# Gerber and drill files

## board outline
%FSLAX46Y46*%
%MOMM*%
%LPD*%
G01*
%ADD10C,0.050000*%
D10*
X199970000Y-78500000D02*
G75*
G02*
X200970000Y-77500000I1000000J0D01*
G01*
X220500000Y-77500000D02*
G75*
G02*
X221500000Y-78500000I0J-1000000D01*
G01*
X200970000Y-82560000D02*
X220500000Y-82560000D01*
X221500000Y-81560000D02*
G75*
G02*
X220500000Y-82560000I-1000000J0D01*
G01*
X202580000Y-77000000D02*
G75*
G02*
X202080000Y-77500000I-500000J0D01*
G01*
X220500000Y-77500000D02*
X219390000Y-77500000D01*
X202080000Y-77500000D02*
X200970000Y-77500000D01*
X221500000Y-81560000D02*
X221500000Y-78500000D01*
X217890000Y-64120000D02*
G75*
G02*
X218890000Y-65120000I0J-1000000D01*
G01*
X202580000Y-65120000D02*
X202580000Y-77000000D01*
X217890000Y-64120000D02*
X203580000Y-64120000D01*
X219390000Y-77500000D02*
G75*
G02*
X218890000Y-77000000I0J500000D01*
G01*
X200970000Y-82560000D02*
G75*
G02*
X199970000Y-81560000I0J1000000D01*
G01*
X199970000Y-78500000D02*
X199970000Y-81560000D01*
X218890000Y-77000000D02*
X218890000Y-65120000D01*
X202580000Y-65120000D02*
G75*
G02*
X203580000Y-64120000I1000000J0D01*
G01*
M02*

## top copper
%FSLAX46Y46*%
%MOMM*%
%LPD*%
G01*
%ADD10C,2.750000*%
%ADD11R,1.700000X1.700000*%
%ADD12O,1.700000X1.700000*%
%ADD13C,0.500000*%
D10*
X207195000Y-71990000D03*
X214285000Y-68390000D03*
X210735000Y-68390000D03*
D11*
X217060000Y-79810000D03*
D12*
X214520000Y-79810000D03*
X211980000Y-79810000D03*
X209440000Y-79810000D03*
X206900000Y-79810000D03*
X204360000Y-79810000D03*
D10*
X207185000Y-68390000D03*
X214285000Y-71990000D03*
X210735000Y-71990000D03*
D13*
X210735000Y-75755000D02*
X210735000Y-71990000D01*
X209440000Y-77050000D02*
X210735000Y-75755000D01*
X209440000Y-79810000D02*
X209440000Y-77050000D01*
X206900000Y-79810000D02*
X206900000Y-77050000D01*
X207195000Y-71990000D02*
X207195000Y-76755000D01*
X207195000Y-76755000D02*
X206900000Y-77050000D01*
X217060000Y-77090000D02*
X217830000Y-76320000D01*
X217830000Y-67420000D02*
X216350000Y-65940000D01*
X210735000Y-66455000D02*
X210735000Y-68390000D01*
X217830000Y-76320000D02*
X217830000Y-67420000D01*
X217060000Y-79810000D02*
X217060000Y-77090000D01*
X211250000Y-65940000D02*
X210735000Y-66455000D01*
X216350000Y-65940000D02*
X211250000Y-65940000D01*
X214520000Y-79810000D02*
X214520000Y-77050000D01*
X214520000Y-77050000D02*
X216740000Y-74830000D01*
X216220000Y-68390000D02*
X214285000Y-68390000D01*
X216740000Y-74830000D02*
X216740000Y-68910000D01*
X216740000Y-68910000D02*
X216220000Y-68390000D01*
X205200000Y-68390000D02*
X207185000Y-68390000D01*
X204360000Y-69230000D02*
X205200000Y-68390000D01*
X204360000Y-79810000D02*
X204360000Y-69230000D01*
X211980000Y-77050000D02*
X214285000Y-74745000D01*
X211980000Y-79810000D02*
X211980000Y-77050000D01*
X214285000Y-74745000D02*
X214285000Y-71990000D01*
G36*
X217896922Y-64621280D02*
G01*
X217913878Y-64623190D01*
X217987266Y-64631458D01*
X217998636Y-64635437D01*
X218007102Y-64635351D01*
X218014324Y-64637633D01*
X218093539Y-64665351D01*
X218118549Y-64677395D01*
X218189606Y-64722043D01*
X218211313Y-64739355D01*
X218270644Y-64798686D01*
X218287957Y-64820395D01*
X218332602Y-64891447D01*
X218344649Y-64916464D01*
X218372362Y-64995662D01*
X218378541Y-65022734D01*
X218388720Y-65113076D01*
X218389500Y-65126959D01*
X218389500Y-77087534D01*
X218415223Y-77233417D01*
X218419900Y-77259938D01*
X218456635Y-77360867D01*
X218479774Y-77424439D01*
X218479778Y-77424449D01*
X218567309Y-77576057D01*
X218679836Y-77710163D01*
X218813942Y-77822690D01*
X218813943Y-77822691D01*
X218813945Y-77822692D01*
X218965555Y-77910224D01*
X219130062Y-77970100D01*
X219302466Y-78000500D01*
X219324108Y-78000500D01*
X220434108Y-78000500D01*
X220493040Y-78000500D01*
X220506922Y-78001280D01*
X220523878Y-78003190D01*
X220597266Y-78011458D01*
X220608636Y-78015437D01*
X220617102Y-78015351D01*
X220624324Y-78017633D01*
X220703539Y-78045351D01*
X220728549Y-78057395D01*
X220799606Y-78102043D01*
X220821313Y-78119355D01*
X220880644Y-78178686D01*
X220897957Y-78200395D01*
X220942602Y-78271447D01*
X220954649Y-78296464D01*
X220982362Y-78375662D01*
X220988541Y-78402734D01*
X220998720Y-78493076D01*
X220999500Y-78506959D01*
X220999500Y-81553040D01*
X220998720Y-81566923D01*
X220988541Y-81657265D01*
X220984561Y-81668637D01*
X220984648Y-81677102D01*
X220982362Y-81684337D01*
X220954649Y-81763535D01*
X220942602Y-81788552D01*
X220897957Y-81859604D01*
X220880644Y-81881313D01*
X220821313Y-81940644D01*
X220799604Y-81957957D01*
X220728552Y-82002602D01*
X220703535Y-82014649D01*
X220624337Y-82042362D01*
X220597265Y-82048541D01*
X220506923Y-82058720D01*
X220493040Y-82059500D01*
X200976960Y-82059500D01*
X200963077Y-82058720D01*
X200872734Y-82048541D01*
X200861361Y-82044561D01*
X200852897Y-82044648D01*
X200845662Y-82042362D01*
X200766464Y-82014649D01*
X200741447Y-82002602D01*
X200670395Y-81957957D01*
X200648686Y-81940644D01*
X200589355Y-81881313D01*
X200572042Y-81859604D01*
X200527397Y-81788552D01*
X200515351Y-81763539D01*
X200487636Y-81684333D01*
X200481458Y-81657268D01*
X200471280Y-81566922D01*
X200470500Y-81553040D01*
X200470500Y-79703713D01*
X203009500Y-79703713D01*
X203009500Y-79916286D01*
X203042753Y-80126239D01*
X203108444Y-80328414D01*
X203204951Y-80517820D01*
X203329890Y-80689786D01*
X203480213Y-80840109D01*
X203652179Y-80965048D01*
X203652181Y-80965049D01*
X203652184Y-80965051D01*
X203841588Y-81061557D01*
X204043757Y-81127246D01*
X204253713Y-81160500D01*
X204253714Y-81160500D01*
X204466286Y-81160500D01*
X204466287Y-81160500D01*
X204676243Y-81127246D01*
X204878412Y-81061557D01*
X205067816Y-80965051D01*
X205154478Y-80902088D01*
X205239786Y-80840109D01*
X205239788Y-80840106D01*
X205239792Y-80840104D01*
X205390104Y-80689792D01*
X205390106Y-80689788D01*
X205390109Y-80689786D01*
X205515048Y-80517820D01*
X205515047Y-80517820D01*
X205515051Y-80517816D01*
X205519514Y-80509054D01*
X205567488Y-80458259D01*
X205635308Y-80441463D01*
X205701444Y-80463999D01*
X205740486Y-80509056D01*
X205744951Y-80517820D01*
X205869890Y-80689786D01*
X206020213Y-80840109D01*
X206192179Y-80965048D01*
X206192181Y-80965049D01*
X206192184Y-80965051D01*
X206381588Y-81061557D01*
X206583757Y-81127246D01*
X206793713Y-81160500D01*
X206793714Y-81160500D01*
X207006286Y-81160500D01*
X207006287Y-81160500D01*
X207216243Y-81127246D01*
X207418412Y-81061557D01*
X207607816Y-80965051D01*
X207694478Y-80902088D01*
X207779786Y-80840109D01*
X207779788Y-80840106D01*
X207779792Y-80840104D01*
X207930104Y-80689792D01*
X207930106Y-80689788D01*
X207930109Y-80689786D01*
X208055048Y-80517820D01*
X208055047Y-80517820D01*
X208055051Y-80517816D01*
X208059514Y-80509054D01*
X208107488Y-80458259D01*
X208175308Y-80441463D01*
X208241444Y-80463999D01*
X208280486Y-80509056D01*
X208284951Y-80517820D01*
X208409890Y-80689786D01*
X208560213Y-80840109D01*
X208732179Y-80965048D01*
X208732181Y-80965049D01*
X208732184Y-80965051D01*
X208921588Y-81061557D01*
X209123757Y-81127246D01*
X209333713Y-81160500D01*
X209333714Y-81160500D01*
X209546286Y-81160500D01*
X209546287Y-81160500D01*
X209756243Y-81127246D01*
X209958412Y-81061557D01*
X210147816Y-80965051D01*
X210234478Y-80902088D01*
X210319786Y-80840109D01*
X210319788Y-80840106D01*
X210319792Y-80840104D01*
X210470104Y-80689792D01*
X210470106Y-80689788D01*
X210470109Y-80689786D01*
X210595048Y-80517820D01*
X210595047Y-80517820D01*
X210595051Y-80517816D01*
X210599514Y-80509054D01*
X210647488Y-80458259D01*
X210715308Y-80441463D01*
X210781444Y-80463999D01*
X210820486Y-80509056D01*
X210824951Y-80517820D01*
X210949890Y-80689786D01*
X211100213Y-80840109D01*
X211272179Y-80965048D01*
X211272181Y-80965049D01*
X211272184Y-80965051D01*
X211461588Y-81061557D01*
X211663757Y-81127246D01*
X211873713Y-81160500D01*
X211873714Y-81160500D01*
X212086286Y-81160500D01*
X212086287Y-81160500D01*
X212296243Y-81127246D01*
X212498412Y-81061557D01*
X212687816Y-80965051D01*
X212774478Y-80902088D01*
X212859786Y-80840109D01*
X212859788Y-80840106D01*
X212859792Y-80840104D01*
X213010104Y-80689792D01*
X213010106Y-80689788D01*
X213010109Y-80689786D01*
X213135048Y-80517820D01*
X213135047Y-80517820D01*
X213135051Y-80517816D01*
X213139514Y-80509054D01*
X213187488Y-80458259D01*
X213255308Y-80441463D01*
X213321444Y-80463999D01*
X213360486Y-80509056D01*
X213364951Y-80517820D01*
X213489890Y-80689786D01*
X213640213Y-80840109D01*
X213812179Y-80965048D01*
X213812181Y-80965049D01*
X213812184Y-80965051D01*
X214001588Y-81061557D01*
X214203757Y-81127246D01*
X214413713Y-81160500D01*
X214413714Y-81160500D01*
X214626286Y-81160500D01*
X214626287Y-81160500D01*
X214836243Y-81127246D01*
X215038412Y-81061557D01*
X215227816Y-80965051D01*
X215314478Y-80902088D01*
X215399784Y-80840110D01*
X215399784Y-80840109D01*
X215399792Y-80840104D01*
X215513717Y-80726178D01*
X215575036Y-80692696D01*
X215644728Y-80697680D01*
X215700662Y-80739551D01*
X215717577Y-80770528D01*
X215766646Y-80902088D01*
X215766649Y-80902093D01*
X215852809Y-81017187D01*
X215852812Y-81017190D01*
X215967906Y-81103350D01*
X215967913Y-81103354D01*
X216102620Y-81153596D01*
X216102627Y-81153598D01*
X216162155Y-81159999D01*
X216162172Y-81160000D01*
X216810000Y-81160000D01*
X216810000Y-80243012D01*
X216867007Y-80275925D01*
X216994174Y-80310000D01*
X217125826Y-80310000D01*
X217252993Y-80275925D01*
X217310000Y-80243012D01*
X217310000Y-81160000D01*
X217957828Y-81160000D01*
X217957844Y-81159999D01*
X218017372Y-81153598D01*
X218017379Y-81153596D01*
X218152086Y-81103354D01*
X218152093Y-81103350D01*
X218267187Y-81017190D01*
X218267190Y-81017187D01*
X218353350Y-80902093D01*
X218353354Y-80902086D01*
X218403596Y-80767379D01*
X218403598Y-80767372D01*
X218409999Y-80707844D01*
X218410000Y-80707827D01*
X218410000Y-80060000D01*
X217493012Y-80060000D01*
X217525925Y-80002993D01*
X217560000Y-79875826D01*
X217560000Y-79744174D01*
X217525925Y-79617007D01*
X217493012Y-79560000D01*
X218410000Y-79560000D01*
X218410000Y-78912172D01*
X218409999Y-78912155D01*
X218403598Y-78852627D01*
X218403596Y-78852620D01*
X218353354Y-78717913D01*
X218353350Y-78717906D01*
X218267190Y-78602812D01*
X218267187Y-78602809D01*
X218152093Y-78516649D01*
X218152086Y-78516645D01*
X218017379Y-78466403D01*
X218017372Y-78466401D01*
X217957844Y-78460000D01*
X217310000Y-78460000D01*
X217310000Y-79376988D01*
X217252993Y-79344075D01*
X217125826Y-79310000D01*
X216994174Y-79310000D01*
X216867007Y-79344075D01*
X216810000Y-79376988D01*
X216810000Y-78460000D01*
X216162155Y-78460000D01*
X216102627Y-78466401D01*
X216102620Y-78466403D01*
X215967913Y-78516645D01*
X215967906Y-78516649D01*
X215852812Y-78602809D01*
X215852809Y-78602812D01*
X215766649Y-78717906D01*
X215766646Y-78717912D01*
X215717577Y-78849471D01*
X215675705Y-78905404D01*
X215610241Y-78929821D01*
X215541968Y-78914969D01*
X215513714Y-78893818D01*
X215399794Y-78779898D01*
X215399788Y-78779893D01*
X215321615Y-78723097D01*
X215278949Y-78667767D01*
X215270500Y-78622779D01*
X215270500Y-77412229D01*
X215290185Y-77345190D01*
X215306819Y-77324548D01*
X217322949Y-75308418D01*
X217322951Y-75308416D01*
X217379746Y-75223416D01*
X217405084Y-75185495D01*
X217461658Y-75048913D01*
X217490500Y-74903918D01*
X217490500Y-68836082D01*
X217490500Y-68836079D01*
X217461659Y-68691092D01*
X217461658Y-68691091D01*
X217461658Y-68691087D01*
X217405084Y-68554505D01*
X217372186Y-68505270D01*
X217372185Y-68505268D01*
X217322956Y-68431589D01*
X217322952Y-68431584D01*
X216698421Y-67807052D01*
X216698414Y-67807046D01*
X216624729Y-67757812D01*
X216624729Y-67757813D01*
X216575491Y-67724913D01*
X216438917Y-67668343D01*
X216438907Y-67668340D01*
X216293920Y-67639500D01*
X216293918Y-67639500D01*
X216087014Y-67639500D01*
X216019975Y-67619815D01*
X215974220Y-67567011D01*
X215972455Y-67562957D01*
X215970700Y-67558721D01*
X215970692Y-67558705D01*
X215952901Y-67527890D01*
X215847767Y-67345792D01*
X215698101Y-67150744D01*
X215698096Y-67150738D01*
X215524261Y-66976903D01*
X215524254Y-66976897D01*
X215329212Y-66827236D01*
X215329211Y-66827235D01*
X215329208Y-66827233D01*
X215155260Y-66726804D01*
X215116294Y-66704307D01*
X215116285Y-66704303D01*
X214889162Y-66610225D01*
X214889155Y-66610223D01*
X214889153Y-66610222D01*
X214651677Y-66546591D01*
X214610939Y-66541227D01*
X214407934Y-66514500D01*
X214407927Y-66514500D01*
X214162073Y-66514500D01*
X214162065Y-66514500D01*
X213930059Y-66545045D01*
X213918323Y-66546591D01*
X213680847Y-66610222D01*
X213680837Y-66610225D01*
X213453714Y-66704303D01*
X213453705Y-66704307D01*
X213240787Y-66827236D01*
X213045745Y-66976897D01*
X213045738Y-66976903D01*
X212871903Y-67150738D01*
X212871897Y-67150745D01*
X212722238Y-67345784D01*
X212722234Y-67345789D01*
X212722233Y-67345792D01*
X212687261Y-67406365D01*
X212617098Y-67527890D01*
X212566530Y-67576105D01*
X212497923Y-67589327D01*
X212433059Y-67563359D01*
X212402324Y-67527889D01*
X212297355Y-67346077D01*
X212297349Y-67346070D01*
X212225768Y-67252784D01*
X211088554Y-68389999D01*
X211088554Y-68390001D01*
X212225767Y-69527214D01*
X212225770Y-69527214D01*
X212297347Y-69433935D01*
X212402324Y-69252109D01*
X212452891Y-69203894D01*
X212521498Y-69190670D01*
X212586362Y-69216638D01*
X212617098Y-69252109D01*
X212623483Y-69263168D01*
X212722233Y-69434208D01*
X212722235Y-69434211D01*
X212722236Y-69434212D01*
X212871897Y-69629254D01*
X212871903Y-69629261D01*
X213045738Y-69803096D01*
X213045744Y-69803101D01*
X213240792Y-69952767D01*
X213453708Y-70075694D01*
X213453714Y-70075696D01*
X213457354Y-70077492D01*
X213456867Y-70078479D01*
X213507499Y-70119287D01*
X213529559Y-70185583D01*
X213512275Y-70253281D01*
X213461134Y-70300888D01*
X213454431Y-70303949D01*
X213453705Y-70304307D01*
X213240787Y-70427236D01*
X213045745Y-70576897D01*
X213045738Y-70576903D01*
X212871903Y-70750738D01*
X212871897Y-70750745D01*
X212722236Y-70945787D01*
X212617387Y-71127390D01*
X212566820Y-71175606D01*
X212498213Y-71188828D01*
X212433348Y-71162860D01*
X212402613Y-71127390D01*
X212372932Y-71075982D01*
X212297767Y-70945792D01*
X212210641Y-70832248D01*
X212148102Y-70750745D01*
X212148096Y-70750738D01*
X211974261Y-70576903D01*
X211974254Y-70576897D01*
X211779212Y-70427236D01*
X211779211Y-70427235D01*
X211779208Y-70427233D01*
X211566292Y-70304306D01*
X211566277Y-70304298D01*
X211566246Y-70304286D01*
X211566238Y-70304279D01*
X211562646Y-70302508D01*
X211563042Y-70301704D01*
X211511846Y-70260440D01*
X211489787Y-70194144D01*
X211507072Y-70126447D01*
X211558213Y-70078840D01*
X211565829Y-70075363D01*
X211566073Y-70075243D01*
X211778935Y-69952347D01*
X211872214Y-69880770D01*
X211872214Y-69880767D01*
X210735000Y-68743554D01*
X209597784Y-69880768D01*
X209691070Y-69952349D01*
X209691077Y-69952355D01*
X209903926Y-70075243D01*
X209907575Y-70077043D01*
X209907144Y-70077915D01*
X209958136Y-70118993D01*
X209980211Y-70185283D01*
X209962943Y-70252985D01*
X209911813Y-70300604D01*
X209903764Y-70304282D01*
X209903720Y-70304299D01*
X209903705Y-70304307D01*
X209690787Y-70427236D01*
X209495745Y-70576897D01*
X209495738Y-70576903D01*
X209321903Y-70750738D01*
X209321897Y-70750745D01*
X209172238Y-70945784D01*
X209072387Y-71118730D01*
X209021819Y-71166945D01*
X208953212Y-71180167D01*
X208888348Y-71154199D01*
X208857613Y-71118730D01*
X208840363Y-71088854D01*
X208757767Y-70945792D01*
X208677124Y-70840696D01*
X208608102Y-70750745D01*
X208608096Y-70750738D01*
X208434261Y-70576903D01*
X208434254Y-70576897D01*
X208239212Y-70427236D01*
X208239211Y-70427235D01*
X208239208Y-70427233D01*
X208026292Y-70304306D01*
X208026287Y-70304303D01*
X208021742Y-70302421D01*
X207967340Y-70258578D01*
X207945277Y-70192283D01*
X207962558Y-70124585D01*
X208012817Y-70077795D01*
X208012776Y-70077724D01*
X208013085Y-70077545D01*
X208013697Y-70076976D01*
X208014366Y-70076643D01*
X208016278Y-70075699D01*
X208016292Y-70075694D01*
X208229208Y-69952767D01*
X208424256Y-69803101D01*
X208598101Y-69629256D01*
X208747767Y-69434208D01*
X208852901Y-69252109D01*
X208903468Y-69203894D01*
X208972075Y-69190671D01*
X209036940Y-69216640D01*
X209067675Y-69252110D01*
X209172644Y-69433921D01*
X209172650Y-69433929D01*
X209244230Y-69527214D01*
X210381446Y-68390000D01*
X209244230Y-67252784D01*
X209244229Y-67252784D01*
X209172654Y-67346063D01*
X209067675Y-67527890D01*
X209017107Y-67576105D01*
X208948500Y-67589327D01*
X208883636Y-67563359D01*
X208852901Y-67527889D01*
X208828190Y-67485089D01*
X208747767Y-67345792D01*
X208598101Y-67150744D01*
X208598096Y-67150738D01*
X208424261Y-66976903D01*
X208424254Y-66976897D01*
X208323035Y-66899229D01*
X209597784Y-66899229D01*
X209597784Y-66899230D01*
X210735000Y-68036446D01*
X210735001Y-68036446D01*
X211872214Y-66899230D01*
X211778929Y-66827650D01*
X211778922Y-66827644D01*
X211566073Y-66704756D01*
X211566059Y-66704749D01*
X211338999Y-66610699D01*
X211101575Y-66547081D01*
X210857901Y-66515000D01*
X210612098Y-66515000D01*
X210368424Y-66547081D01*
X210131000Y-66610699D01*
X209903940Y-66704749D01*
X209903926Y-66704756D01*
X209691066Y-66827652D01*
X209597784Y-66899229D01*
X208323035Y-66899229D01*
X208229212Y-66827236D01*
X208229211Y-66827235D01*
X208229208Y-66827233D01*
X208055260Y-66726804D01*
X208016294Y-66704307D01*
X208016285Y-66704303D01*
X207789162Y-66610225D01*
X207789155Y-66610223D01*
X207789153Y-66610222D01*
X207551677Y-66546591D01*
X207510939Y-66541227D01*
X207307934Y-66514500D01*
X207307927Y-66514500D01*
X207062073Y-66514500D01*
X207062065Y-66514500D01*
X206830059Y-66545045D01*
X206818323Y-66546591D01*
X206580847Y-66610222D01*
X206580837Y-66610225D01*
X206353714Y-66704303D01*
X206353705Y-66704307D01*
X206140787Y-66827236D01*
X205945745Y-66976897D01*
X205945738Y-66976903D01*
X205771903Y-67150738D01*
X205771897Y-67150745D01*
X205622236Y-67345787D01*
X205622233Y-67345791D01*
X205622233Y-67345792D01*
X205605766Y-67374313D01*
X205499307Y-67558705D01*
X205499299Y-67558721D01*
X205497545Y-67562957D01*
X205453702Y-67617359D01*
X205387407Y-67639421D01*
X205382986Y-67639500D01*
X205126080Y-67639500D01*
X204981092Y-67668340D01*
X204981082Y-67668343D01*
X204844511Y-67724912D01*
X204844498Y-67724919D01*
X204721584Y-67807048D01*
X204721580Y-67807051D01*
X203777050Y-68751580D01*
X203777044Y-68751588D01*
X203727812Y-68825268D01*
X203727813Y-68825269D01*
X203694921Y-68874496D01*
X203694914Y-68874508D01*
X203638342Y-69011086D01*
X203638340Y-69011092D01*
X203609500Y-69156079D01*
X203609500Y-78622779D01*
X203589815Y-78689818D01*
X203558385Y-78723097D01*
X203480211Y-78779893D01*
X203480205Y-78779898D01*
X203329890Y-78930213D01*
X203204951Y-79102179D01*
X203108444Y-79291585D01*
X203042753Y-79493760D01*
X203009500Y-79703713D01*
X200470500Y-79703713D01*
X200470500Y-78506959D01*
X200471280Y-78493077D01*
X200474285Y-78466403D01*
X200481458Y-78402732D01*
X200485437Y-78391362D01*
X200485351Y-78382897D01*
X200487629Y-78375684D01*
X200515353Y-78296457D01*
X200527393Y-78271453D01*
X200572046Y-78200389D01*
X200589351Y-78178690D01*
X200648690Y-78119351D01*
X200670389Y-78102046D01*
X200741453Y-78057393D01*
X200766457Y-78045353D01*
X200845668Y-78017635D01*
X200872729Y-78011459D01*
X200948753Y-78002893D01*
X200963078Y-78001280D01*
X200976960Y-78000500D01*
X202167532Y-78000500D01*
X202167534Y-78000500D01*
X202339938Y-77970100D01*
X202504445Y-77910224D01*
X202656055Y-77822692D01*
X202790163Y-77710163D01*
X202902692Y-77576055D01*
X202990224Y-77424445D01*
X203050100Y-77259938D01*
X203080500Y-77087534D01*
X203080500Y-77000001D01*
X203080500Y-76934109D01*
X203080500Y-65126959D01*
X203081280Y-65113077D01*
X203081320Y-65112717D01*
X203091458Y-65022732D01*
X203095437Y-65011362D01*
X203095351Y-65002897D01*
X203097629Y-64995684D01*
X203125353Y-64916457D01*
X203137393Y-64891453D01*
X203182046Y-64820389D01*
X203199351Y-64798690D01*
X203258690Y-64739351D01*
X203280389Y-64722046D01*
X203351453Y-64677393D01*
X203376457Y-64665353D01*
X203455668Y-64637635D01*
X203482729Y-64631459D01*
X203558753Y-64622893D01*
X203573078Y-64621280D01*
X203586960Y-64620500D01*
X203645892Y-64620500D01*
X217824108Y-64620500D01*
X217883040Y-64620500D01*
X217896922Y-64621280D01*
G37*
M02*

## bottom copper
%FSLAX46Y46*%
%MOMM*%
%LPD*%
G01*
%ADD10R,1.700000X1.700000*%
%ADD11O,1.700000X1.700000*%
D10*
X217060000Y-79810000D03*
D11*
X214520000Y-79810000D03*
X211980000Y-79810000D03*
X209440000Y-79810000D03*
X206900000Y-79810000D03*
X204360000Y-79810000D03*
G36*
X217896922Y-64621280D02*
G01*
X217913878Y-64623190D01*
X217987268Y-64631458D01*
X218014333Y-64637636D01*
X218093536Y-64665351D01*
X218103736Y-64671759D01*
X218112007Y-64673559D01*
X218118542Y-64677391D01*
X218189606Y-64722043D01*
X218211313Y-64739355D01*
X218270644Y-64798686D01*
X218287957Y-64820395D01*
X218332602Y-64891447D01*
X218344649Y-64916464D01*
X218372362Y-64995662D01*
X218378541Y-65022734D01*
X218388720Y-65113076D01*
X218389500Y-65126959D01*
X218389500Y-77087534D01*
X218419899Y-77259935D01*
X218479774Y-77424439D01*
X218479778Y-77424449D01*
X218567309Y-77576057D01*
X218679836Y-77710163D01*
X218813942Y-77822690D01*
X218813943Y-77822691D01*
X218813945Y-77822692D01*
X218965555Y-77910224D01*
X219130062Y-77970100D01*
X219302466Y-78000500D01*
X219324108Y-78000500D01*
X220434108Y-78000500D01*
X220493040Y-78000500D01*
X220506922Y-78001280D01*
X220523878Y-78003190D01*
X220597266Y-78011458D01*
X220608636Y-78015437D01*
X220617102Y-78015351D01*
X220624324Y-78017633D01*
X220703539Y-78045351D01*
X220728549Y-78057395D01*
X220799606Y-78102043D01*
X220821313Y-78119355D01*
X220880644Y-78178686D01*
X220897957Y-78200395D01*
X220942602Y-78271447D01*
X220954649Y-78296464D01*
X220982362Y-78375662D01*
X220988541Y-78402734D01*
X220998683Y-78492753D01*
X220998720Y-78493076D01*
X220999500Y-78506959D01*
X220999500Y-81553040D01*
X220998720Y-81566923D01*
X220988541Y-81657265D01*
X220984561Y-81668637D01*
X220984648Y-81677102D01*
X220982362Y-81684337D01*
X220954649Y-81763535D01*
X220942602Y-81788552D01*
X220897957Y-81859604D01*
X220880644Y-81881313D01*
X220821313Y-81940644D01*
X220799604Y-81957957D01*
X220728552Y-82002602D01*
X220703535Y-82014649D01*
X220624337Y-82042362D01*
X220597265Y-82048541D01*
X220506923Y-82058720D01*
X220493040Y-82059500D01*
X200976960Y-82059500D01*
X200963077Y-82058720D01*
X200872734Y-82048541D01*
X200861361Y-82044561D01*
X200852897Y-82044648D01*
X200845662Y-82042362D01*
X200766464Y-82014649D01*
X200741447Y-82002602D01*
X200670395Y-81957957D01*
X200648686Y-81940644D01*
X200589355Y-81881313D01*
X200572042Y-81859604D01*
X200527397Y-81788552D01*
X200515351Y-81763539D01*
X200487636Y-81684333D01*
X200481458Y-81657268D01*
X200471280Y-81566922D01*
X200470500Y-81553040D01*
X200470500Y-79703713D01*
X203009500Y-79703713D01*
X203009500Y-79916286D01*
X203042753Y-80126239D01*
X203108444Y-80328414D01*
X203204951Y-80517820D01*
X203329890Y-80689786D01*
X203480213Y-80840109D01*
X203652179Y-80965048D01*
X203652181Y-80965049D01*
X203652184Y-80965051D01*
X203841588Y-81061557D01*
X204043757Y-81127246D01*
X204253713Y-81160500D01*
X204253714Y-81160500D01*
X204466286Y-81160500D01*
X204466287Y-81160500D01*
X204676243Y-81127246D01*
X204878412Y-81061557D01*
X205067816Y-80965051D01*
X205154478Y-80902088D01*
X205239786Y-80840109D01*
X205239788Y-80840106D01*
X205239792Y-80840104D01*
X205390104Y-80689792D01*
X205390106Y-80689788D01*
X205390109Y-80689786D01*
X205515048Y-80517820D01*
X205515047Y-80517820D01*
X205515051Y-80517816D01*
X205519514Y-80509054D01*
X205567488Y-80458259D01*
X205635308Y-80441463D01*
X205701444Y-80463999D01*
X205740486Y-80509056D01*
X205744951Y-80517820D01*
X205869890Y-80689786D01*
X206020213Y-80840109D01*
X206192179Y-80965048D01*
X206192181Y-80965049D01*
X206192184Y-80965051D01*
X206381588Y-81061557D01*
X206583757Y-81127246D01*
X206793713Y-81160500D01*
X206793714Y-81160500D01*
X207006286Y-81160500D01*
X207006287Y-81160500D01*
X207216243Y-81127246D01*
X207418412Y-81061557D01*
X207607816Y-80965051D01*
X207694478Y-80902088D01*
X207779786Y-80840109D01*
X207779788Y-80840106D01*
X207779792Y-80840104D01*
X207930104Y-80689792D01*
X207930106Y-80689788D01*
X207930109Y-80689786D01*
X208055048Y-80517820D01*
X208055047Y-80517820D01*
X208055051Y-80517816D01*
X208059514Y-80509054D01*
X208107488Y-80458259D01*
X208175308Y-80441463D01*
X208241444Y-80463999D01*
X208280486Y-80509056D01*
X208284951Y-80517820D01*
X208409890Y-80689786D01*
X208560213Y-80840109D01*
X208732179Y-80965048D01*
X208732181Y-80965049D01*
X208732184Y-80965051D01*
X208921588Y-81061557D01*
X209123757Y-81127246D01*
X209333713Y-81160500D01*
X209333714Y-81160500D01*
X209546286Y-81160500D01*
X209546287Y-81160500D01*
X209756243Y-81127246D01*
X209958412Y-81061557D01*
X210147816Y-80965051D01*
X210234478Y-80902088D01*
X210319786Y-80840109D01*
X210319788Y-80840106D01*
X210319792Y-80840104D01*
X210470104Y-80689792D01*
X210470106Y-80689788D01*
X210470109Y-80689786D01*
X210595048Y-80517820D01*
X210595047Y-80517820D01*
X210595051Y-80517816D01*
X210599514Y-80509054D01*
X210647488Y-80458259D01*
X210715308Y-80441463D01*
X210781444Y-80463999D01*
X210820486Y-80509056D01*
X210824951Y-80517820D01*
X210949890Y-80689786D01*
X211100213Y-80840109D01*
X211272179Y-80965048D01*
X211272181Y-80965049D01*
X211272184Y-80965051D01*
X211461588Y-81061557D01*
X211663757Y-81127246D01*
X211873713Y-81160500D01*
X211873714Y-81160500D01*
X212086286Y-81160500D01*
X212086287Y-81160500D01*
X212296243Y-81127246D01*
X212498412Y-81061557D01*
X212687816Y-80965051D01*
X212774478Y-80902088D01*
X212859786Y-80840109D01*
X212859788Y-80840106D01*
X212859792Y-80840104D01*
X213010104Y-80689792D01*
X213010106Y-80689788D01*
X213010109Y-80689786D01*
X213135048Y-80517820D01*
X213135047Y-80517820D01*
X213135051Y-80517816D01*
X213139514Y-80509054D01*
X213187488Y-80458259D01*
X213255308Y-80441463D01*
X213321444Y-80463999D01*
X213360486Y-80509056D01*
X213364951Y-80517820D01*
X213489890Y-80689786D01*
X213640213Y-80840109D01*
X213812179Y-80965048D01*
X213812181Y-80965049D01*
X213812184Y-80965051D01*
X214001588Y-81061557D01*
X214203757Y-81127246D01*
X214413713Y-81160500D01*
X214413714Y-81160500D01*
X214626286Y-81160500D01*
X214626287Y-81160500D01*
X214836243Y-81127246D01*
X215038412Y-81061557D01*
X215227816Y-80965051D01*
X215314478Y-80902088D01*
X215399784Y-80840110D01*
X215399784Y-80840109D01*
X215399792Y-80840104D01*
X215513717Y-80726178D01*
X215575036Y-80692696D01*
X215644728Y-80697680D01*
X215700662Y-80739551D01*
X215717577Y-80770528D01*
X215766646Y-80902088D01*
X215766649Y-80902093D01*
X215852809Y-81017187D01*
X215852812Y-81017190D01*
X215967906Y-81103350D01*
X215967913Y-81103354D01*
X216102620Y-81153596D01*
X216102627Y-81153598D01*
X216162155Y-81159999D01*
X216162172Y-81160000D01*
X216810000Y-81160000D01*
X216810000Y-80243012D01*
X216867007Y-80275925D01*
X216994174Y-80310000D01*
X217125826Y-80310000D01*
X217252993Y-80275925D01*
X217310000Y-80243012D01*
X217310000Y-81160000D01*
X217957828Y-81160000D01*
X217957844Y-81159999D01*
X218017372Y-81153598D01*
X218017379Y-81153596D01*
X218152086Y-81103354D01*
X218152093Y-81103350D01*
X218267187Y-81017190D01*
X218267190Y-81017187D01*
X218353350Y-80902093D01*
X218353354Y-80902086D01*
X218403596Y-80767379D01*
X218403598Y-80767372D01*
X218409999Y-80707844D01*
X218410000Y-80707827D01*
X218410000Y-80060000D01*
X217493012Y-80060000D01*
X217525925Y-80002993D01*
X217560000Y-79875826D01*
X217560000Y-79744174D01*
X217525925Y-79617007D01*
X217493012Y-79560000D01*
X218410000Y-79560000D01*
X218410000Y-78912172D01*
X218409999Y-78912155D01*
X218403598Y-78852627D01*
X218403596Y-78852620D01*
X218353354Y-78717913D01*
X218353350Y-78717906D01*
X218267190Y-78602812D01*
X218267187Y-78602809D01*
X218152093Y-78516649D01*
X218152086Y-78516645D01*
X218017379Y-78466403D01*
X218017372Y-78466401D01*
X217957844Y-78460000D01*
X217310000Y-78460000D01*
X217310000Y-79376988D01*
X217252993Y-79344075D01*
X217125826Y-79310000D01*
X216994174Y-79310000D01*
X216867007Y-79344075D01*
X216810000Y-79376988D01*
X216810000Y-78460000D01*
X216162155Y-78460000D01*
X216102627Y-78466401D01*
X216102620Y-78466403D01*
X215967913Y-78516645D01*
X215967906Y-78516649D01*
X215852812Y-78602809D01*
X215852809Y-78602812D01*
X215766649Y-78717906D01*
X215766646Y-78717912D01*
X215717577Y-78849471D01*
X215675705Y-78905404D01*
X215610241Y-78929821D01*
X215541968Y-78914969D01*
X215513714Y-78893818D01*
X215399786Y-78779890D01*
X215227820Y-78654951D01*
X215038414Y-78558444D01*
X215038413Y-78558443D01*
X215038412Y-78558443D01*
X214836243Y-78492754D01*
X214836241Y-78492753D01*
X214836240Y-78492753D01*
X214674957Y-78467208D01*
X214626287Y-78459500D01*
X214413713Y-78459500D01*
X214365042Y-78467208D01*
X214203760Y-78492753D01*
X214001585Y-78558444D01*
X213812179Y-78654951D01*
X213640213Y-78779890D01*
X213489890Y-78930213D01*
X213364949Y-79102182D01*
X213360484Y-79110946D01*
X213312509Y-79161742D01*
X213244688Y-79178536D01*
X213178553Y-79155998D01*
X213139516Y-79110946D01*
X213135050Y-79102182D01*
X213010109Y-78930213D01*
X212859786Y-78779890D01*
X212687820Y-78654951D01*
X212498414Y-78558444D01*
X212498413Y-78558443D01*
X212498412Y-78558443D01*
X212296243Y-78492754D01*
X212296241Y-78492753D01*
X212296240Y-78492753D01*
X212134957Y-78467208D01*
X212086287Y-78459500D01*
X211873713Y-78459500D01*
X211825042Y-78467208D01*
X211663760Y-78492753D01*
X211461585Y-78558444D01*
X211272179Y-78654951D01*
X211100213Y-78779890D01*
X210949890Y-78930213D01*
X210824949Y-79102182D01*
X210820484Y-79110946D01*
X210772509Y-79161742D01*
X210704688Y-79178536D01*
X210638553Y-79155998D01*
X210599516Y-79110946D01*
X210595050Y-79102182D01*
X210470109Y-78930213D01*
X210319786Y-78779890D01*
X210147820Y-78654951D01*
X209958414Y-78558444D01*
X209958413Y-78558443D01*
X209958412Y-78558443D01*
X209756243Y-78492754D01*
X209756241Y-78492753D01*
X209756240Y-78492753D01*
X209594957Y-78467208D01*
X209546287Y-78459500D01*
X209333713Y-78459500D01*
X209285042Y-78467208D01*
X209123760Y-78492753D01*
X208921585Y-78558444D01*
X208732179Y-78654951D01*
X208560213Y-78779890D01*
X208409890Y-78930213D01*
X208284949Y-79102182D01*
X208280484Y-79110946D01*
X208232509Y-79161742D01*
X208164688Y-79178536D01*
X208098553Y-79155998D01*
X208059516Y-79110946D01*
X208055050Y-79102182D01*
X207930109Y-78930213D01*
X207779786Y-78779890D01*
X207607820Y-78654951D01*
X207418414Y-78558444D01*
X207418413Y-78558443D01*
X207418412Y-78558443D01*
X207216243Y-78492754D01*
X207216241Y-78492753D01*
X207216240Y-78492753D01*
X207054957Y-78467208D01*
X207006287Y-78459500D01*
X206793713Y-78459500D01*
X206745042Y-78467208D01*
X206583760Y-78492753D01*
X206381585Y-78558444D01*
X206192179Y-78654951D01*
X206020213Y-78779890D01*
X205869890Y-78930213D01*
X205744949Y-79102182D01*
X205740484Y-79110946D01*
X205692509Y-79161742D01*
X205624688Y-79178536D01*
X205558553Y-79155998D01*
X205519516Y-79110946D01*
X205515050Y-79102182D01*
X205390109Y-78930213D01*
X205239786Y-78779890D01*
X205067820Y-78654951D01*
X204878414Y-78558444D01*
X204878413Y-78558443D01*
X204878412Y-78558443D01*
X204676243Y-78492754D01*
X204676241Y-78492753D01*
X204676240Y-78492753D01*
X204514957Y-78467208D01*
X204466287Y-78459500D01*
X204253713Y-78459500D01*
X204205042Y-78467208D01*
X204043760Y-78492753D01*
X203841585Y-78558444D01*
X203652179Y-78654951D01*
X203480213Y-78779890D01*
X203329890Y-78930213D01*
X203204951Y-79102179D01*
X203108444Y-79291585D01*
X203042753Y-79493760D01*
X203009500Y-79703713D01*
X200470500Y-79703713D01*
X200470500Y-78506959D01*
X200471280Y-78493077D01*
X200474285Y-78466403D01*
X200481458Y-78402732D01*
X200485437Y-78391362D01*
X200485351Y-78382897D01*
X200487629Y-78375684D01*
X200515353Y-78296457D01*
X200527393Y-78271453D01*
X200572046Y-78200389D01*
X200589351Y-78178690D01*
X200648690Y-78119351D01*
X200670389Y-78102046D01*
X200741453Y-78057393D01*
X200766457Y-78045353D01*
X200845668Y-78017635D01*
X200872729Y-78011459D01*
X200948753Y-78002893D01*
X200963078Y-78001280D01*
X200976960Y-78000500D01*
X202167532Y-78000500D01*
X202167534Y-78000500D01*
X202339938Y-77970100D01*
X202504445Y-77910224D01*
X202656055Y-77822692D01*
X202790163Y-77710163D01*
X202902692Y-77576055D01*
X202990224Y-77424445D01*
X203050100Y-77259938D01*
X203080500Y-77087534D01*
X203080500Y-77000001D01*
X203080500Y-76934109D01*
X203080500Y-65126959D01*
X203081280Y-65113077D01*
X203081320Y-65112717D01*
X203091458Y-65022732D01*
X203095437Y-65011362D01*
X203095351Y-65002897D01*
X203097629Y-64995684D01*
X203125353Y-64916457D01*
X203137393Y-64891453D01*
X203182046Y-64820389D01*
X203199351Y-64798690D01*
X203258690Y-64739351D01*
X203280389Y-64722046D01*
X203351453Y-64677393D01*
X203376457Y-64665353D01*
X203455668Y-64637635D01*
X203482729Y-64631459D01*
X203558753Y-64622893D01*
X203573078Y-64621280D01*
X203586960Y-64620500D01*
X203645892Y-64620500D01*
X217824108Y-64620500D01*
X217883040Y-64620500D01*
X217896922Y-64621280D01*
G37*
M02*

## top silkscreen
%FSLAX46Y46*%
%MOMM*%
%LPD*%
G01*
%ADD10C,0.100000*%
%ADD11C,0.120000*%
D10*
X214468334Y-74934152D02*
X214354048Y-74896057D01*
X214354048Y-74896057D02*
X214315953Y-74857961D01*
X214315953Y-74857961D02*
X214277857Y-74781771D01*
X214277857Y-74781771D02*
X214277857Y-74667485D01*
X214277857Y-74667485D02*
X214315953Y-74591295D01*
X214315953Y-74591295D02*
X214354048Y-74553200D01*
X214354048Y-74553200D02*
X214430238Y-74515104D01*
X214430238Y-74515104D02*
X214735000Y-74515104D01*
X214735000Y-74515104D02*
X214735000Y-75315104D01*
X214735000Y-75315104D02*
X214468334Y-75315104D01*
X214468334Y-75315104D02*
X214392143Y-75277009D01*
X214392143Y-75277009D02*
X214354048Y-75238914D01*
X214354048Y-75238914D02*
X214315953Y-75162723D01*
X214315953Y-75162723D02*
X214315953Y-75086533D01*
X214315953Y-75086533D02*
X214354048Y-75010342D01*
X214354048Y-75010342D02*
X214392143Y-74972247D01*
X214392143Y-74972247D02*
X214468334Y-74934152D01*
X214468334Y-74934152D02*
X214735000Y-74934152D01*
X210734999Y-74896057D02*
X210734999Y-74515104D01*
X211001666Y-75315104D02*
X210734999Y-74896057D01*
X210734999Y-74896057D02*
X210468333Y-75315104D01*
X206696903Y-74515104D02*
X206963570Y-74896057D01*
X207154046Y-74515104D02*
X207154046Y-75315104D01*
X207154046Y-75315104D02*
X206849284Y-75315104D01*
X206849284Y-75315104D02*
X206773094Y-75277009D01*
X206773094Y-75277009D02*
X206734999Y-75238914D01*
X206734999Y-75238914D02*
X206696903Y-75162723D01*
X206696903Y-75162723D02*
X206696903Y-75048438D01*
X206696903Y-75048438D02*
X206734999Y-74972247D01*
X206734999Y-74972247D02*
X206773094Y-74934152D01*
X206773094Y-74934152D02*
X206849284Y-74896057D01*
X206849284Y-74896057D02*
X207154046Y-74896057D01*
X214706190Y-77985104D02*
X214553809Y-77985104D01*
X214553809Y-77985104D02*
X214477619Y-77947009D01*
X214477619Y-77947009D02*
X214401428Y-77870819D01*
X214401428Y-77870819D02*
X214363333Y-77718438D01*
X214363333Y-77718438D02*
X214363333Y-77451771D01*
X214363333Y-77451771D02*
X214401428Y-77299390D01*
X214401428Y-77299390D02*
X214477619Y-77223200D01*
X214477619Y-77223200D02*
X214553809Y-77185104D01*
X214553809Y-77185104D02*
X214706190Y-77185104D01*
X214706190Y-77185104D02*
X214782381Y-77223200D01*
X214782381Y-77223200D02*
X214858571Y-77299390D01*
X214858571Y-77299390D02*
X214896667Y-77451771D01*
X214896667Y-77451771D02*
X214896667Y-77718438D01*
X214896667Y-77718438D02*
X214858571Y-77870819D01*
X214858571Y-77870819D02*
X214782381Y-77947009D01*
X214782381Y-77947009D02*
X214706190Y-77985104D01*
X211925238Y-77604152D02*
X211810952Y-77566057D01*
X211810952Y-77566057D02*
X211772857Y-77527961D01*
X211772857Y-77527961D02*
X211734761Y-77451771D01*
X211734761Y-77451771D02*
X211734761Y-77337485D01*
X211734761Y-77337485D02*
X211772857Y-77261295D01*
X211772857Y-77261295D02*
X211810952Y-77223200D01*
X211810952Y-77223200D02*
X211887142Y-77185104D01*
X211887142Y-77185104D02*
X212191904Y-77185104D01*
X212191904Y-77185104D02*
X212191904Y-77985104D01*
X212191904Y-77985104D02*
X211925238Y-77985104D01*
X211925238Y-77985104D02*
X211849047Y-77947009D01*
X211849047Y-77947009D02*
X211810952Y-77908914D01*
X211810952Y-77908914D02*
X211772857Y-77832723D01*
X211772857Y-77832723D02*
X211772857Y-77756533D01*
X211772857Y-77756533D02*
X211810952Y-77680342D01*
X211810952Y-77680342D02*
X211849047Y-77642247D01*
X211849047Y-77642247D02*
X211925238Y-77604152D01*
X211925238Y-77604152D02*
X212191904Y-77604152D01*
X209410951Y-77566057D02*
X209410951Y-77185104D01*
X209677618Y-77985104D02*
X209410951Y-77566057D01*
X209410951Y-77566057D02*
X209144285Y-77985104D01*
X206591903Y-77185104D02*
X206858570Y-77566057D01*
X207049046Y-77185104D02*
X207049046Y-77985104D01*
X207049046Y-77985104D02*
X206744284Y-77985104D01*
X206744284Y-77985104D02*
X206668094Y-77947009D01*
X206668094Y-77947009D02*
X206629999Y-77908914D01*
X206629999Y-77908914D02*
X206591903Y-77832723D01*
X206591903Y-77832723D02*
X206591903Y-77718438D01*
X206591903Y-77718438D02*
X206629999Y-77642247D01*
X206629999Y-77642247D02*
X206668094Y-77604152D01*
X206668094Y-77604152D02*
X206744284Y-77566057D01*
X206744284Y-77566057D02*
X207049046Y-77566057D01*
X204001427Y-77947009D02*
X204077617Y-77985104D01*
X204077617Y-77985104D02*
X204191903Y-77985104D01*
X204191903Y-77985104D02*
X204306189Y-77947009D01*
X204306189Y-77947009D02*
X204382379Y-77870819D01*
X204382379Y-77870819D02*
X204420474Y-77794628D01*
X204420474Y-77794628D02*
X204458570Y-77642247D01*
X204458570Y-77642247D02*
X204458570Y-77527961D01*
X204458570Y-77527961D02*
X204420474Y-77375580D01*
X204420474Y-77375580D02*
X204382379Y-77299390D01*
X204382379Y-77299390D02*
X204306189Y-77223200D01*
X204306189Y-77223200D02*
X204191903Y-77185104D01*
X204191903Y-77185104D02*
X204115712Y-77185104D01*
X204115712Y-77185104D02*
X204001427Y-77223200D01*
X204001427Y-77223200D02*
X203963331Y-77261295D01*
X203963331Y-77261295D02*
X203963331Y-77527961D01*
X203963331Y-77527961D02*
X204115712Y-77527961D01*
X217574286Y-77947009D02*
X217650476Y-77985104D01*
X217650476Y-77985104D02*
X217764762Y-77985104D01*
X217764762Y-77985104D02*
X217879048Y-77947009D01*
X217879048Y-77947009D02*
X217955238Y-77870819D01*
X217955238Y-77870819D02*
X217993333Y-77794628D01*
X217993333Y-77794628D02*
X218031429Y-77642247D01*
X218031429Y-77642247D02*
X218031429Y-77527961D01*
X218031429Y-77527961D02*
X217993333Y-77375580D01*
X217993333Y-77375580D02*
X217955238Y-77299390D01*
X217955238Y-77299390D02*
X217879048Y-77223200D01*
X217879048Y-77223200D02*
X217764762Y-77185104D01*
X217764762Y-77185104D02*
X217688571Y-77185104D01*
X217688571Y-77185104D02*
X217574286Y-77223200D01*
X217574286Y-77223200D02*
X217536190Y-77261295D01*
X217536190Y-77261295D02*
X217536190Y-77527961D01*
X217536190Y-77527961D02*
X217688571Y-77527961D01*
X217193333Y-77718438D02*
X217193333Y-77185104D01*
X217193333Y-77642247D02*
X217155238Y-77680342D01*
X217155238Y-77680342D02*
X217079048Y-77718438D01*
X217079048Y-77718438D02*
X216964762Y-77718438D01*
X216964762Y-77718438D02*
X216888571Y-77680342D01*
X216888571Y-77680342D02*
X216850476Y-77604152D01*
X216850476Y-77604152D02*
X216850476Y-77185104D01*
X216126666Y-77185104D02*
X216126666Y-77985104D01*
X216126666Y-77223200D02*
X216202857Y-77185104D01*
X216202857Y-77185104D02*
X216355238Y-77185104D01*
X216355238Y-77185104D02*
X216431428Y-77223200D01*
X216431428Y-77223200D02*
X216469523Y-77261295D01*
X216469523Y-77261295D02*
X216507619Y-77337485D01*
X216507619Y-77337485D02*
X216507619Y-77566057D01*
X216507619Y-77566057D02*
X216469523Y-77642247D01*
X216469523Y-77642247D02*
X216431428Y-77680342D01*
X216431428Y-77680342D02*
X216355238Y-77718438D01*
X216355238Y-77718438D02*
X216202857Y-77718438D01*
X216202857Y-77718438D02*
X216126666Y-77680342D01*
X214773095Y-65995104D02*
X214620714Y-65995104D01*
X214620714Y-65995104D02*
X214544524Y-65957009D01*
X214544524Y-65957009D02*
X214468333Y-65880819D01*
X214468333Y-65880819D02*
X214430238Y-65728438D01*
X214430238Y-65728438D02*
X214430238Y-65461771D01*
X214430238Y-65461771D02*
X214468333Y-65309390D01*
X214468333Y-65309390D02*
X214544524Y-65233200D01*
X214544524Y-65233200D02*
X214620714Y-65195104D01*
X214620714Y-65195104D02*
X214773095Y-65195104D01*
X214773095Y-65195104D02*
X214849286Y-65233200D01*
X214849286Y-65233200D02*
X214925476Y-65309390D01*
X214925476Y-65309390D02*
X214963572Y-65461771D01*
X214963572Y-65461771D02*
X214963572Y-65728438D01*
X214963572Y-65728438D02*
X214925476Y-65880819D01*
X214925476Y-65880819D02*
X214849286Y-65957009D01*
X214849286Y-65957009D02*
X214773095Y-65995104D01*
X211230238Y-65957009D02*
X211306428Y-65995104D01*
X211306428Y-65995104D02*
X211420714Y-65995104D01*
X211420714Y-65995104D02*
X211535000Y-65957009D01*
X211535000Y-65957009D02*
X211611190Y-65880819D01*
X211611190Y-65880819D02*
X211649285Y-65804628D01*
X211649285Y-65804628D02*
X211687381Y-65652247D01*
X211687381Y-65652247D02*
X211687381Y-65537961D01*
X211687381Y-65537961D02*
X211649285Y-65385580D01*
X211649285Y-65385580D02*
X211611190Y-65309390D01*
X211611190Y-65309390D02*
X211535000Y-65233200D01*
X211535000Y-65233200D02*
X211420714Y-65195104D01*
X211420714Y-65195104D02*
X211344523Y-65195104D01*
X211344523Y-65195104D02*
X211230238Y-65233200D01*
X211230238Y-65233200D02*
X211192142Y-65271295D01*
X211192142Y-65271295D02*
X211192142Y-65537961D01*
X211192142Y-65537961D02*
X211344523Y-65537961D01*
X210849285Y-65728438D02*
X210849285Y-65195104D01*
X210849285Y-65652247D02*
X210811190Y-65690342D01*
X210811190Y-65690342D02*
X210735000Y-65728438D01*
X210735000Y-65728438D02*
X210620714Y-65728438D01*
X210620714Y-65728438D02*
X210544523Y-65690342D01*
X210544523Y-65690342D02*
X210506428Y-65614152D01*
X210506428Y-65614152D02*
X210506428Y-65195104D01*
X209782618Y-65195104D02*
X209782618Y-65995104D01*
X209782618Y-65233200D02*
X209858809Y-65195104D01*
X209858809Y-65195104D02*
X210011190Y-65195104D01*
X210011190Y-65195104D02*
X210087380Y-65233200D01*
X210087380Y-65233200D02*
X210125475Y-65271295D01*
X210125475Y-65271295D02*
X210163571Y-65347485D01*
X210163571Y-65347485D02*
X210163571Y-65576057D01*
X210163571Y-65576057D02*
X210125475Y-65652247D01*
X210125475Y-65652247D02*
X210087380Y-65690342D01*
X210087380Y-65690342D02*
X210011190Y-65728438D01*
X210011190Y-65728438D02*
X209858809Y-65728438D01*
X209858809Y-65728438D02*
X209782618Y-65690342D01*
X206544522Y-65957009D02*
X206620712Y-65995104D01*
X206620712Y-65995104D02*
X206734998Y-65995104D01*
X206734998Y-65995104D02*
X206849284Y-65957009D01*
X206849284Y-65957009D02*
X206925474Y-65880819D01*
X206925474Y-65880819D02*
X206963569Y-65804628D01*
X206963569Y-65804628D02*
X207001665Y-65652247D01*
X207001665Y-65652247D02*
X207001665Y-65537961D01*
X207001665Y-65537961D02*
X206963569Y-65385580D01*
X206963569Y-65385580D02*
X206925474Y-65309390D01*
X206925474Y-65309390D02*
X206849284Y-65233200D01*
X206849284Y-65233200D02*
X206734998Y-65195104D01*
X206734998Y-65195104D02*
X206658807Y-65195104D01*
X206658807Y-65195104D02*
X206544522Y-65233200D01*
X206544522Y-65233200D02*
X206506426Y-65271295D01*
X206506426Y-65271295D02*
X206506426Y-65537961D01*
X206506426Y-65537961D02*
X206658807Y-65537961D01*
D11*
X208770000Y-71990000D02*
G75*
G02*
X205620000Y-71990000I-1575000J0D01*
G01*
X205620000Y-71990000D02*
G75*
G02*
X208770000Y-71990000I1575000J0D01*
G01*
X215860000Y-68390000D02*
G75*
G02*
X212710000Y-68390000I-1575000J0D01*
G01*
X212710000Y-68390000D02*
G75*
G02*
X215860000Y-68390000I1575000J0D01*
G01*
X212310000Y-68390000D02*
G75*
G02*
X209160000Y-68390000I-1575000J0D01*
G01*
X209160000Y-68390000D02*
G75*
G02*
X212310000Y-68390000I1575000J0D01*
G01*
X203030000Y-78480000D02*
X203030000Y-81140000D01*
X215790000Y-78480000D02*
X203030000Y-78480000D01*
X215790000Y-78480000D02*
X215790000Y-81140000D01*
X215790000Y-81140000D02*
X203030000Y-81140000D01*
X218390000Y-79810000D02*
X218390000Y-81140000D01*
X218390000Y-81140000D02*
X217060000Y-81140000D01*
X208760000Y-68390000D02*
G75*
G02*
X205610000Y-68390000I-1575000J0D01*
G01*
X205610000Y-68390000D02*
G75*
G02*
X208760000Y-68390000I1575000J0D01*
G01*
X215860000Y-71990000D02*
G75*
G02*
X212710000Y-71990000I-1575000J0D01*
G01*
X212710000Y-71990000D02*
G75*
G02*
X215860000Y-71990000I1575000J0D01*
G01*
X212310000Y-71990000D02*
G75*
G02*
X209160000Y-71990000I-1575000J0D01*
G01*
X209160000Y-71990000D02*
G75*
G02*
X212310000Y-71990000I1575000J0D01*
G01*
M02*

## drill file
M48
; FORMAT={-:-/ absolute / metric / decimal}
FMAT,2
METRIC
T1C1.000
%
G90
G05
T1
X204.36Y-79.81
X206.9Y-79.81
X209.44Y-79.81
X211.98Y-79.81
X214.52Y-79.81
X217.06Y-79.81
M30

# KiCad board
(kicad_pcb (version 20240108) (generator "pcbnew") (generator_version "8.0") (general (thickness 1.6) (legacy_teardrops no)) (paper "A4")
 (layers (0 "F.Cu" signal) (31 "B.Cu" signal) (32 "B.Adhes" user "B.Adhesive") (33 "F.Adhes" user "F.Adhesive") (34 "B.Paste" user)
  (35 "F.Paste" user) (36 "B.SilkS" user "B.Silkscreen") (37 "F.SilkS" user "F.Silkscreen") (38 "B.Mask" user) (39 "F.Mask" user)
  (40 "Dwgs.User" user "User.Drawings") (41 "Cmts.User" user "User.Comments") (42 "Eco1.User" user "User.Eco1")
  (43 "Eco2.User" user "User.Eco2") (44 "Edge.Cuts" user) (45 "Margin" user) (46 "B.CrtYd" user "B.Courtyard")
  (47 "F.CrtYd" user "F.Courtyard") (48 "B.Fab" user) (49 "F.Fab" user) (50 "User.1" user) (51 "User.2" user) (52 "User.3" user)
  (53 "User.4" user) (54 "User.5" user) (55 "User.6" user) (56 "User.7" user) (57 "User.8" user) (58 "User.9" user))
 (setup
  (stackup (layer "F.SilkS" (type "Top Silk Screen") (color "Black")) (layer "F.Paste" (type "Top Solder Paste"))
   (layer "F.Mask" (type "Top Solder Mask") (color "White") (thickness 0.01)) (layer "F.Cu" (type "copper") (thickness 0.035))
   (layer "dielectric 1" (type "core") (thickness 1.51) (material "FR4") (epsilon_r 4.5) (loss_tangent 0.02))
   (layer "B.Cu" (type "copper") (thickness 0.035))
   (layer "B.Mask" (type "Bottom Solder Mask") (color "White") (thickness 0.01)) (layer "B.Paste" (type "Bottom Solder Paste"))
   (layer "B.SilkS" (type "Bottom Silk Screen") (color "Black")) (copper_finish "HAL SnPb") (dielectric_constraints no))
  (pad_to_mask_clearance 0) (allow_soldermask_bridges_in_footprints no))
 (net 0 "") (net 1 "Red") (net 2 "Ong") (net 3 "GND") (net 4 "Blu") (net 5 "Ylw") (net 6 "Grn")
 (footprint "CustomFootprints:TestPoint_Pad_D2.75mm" (layer "F.Cu") (at 207.195 71.99)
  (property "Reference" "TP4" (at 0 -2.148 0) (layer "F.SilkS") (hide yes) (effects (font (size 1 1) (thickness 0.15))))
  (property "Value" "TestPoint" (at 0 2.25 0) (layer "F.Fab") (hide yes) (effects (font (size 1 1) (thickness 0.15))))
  (fp_circle (center 0 0) (end 1.575 0) (stroke (width 0.12) (type solid)) (fill none) (layer "F.SilkS"))
  (pad "1" smd circle (at 0 0) (size 2.75 2.75) (layers "F.Cu" "F.Mask") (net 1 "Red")))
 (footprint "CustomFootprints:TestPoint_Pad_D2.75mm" (layer "F.Cu") (at 214.285 68.39)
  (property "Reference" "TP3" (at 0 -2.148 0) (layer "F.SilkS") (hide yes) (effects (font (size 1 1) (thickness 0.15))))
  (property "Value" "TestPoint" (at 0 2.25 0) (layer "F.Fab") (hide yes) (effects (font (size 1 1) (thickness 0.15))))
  (fp_circle (center 0 0) (end 1.575 0) (stroke (width 0.12) (type solid)) (fill none) (layer "F.SilkS"))
  (pad "1" smd circle (at 0 0) (size 2.75 2.75) (layers "F.Cu" "F.Mask") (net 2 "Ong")))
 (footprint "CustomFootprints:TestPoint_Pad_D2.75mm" (layer "F.Cu") (at 210.735 68.39)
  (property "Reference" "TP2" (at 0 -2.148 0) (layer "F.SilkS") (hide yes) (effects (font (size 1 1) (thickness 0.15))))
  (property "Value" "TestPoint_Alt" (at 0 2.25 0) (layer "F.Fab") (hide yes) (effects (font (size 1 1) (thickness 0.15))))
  (fp_circle (center 0 0) (end 1.575 0) (stroke (width 0.12) (type solid)) (fill none) (layer "F.SilkS"))
  (pad "1" smd circle (at 0 0) (size 2.75 2.75) (layers "F.Cu" "F.Mask") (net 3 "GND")))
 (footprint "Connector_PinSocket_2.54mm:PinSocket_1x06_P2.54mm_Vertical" (layer "F.Cu") (at 217.06 79.81 -90)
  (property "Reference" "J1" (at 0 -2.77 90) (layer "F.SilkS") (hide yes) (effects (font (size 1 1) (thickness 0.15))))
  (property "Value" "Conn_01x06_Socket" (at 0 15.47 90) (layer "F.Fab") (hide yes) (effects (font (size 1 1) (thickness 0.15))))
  (fp_line (start -1.33 14.03) (end 1.33 14.03) (stroke (width 0.12) (type solid)) (layer "F.SilkS"))
  (fp_line (start -1.33 1.27) (end -1.33 14.03) (stroke (width 0.12) (type solid)) (layer "F.SilkS"))
  (fp_line (start -1.33 1.27) (end 1.33 1.27) (stroke (width 0.12) (type solid)) (layer "F.SilkS"))
  (fp_line (start 1.33 1.27) (end 1.33 14.03) (stroke (width 0.12) (type solid)) (layer "F.SilkS"))
  (fp_line (start 0 -1.33) (end 1.33 -1.33) (stroke (width 0.12) (type solid)) (layer "F.SilkS"))
  (fp_line (start 1.33 -1.33) (end 1.33 0) (stroke (width 0.12) (type solid)) (layer "F.SilkS"))
  (pad "1" thru_hole rect (at 0 0 270) (size 1.7 1.7) (drill 1) (layers "*.Cu" "*.Mask") (remove_unused_layers no) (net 3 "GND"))
  (pad "2" thru_hole oval (at 0 2.54 270) (size 1.7 1.7) (drill 1) (layers "*.Cu" "*.Mask") (remove_unused_layers no) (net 2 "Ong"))
  (pad "3" thru_hole oval (at 0 5.08 270) (size 1.7 1.7) (drill 1) (layers "*.Cu" "*.Mask") (remove_unused_layers no) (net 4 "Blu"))
  (pad "4" thru_hole oval (at 0 7.62 270) (size 1.7 1.7) (drill 1) (layers "*.Cu" "*.Mask") (remove_unused_layers no) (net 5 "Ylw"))
  (pad "5" thru_hole oval (at 0 10.16 270) (size 1.7 1.7) (drill 1) (layers "*.Cu" "*.Mask") (remove_unused_layers no) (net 1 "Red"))
  (pad "6" thru_hole oval (at 0 12.7 270) (size 1.7 1.7) (drill 1) (layers "*.Cu" "*.Mask") (remove_unused_layers no) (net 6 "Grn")))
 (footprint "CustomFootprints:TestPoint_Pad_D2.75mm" (layer "F.Cu") (at 207.185 68.39)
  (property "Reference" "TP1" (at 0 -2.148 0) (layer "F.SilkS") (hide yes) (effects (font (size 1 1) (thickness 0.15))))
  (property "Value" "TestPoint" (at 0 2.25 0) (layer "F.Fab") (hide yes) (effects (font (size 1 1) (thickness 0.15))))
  (fp_circle (center 0 0) (end 1.575 0) (stroke (width 0.12) (type solid)) (fill none) (layer "F.SilkS"))
  (pad "1" smd circle (at 0 0) (size 2.75 2.75) (layers "F.Cu" "F.Mask") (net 6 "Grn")))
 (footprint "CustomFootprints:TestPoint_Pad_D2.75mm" (layer "F.Cu") (at 214.285 71.99)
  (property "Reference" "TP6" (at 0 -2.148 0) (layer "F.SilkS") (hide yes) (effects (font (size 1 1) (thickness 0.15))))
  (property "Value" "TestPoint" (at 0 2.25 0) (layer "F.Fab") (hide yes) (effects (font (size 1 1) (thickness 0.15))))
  (fp_circle (center 0 0) (end 1.575 0) (stroke (width 0.12) (type solid)) (fill none) (layer "F.SilkS"))
  (pad "1" smd circle (at 0 0) (size 2.75 2.75) (layers "F.Cu" "F.Mask") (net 4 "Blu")))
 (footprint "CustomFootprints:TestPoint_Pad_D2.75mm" (layer "F.Cu") (at 210.735 71.99)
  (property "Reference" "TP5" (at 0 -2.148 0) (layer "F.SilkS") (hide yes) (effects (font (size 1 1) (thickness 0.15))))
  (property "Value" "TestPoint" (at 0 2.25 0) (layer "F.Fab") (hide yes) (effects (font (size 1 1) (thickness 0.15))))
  (fp_circle (center 0 0) (end 1.575 0) (stroke (width 0.12) (type solid)) (fill none) (layer "F.SilkS"))
  (pad "1" smd circle (at 0 0) (size 2.75 2.75) (layers "F.Cu" "F.Mask") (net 5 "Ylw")))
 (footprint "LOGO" (layer "B.Cu") (at 210.72 71.060277 180)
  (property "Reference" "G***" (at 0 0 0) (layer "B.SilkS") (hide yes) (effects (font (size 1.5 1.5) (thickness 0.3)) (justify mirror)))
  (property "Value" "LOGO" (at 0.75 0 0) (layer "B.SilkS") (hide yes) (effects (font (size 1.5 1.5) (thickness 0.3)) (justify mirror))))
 (gr_arc (start 199.97 78.5) (mid 200.262893 77.792893) (end 200.97 77.5) (stroke (width 0.05) (type default)) (layer "Edge.Cuts"))
 (gr_arc (start 220.5 77.5) (mid 221.207107 77.792893) (end 221.5 78.5) (stroke (width 0.05) (type default)) (layer "Edge.Cuts"))
 (gr_line (start 200.97 82.56) (end 220.5 82.56) (stroke (width 0.05) (type default)) (layer "Edge.Cuts"))
 (gr_arc (start 221.5 81.56) (mid 221.207107 82.267107) (end 220.5 82.56) (stroke (width 0.05) (type default)) (layer "Edge.Cuts"))
 (gr_arc (start 202.58 77) (mid 202.433553 77.353553) (end 202.08 77.5) (stroke (width 0.05) (type default)) (layer "Edge.Cuts"))
 (gr_line (start 220.5 77.5) (end 219.39 77.5) (stroke (width 0.05) (type default)) (layer "Edge.Cuts"))
 (gr_line (start 202.08 77.5) (end 200.97 77.5) (stroke (width 0.05) (type default)) (layer "Edge.Cuts"))
 (gr_line (start 221.5 81.56) (end 221.5 78.5) (stroke (width 0.05) (type default)) (layer "Edge.Cuts"))
 (gr_arc (start 217.89 64.12) (mid 218.597107 64.412893) (end 218.89 65.12) (stroke (width 0.05) (type default)) (layer "Edge.Cuts"))
 (gr_line (start 202.58 65.12) (end 202.58 77) (stroke (width 0.05) (type default)) (layer "Edge.Cuts"))
 (gr_line (start 217.89 64.12) (end 203.58 64.12) (stroke (width 0.05) (type default)) (layer "Edge.Cuts"))
 (gr_arc (start 219.39 77.5) (mid 219.036447 77.353553) (end 218.89 77) (stroke (width 0.05) (type default)) (layer "Edge.Cuts"))
 (gr_arc (start 200.97 82.56) (mid 200.262893 82.267107) (end 199.97 81.56) (stroke (width 0.05) (type default)) (layer "Edge.Cuts"))
 (gr_line (start 199.97 78.5) (end 199.97 81.56) (stroke (width 0.05) (type default)) (layer "Edge.Cuts"))
 (gr_line (start 218.89 77) (end 218.89 65.12) (stroke (width 0.05) (type default)) (layer "Edge.Cuts"))
 (gr_arc (start 202.58 65.12) (mid 202.872893 64.412893) (end 203.58 64.12) (stroke (width 0.05) (type default)) (layer "Edge.Cuts"))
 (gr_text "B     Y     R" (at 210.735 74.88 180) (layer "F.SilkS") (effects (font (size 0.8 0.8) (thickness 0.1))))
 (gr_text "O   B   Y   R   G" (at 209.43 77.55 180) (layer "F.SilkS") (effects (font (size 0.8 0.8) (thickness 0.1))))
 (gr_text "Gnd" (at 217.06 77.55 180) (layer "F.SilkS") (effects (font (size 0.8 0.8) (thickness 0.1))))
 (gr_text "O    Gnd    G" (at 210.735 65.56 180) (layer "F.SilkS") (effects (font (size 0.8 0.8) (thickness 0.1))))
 (segment (start 210.735 75.755) (end 210.735 71.99) (width 0.5) (layer "F.Cu") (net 5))
 (segment (start 209.44 77.05) (end 210.735 75.755) (width 0.5) (layer "F.Cu") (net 5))
 (segment (start 209.44 79.81) (end 209.44 77.05) (width 0.5) (layer "F.Cu") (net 5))
 (segment (start 206.9 79.81) (end 206.9 77.05) (width 0.5) (layer "F.Cu") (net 1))
 (segment (start 207.195 71.99) (end 207.195 76.755) (width 0.5) (layer "F.Cu") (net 1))
 (segment (start 207.195 76.755) (end 206.9 77.05) (width 0.5) (layer "F.Cu") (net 1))
 (segment (start 217.06 77.09) (end 217.83 76.32) (width 0.5) (layer "F.Cu") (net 3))
 (segment (start 217.83 67.42) (end 216.35 65.94) (width 0.5) (layer "F.Cu") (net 3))
 (segment (start 210.735 66.455) (end 210.735 68.39) (width 0.5) (layer "F.Cu") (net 3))
 (segment (start 217.83 76.32) (end 217.83 67.42) (width 0.5) (layer "F.Cu") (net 3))
 (segment (start 217.06 79.81) (end 217.06 77.09) (width 0.5) (layer "F.Cu") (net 3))
 (segment (start 211.25 65.94) (end 210.735 66.455) (width 0.5) (layer "F.Cu") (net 3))
 (segment (start 216.35 65.94) (end 211.25 65.94) (width 0.5) (layer "F.Cu") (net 3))
 (segment (start 214.52 79.81) (end 214.52 77.05) (width 0.5) (layer "F.Cu") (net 2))
 (segment (start 214.52 77.05) (end 216.74 74.83) (width 0.5) (layer "F.Cu") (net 2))
 (segment (start 216.22 68.39) (end 214.285 68.39) (width 0.5) (layer "F.Cu") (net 2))
 (segment (start 216.74 74.83) (end 216.74 68.91) (width 0.5) (layer "F.Cu") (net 2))
 (segment (start 216.74 68.91) (end 216.22 68.39) (width 0.5) (layer "F.Cu") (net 2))
 (segment (start 205.2 68.39) (end 207.185 68.39) (width 0.5) (layer "F.Cu") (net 6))
 (segment (start 204.36 69.23) (end 205.2 68.39) (width 0.5) (layer "F.Cu") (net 6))
 (segment (start 204.36 79.81) (end 204.36 69.23) (width 0.5) (layer "F.Cu") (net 6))
 (segment (start 211.98 77.05) (end 214.285 74.745) (width 0.5) (layer "F.Cu") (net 4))
 (segment (start 211.98 79.81) (end 211.98 77.05) (width 0.5) (layer "F.Cu") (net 4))
 (segment (start 214.285 74.745) (end 214.285 71.99) (width 0.5) (layer "F.Cu") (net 4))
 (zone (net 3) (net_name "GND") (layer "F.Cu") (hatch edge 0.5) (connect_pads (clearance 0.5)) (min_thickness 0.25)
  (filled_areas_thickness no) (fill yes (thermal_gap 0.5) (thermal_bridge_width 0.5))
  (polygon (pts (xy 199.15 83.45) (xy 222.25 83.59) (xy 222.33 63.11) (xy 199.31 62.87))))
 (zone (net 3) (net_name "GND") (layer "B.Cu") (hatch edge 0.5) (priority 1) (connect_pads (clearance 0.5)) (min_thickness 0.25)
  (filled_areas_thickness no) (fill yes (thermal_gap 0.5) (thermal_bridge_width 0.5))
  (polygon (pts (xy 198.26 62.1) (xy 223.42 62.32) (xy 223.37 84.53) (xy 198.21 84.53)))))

